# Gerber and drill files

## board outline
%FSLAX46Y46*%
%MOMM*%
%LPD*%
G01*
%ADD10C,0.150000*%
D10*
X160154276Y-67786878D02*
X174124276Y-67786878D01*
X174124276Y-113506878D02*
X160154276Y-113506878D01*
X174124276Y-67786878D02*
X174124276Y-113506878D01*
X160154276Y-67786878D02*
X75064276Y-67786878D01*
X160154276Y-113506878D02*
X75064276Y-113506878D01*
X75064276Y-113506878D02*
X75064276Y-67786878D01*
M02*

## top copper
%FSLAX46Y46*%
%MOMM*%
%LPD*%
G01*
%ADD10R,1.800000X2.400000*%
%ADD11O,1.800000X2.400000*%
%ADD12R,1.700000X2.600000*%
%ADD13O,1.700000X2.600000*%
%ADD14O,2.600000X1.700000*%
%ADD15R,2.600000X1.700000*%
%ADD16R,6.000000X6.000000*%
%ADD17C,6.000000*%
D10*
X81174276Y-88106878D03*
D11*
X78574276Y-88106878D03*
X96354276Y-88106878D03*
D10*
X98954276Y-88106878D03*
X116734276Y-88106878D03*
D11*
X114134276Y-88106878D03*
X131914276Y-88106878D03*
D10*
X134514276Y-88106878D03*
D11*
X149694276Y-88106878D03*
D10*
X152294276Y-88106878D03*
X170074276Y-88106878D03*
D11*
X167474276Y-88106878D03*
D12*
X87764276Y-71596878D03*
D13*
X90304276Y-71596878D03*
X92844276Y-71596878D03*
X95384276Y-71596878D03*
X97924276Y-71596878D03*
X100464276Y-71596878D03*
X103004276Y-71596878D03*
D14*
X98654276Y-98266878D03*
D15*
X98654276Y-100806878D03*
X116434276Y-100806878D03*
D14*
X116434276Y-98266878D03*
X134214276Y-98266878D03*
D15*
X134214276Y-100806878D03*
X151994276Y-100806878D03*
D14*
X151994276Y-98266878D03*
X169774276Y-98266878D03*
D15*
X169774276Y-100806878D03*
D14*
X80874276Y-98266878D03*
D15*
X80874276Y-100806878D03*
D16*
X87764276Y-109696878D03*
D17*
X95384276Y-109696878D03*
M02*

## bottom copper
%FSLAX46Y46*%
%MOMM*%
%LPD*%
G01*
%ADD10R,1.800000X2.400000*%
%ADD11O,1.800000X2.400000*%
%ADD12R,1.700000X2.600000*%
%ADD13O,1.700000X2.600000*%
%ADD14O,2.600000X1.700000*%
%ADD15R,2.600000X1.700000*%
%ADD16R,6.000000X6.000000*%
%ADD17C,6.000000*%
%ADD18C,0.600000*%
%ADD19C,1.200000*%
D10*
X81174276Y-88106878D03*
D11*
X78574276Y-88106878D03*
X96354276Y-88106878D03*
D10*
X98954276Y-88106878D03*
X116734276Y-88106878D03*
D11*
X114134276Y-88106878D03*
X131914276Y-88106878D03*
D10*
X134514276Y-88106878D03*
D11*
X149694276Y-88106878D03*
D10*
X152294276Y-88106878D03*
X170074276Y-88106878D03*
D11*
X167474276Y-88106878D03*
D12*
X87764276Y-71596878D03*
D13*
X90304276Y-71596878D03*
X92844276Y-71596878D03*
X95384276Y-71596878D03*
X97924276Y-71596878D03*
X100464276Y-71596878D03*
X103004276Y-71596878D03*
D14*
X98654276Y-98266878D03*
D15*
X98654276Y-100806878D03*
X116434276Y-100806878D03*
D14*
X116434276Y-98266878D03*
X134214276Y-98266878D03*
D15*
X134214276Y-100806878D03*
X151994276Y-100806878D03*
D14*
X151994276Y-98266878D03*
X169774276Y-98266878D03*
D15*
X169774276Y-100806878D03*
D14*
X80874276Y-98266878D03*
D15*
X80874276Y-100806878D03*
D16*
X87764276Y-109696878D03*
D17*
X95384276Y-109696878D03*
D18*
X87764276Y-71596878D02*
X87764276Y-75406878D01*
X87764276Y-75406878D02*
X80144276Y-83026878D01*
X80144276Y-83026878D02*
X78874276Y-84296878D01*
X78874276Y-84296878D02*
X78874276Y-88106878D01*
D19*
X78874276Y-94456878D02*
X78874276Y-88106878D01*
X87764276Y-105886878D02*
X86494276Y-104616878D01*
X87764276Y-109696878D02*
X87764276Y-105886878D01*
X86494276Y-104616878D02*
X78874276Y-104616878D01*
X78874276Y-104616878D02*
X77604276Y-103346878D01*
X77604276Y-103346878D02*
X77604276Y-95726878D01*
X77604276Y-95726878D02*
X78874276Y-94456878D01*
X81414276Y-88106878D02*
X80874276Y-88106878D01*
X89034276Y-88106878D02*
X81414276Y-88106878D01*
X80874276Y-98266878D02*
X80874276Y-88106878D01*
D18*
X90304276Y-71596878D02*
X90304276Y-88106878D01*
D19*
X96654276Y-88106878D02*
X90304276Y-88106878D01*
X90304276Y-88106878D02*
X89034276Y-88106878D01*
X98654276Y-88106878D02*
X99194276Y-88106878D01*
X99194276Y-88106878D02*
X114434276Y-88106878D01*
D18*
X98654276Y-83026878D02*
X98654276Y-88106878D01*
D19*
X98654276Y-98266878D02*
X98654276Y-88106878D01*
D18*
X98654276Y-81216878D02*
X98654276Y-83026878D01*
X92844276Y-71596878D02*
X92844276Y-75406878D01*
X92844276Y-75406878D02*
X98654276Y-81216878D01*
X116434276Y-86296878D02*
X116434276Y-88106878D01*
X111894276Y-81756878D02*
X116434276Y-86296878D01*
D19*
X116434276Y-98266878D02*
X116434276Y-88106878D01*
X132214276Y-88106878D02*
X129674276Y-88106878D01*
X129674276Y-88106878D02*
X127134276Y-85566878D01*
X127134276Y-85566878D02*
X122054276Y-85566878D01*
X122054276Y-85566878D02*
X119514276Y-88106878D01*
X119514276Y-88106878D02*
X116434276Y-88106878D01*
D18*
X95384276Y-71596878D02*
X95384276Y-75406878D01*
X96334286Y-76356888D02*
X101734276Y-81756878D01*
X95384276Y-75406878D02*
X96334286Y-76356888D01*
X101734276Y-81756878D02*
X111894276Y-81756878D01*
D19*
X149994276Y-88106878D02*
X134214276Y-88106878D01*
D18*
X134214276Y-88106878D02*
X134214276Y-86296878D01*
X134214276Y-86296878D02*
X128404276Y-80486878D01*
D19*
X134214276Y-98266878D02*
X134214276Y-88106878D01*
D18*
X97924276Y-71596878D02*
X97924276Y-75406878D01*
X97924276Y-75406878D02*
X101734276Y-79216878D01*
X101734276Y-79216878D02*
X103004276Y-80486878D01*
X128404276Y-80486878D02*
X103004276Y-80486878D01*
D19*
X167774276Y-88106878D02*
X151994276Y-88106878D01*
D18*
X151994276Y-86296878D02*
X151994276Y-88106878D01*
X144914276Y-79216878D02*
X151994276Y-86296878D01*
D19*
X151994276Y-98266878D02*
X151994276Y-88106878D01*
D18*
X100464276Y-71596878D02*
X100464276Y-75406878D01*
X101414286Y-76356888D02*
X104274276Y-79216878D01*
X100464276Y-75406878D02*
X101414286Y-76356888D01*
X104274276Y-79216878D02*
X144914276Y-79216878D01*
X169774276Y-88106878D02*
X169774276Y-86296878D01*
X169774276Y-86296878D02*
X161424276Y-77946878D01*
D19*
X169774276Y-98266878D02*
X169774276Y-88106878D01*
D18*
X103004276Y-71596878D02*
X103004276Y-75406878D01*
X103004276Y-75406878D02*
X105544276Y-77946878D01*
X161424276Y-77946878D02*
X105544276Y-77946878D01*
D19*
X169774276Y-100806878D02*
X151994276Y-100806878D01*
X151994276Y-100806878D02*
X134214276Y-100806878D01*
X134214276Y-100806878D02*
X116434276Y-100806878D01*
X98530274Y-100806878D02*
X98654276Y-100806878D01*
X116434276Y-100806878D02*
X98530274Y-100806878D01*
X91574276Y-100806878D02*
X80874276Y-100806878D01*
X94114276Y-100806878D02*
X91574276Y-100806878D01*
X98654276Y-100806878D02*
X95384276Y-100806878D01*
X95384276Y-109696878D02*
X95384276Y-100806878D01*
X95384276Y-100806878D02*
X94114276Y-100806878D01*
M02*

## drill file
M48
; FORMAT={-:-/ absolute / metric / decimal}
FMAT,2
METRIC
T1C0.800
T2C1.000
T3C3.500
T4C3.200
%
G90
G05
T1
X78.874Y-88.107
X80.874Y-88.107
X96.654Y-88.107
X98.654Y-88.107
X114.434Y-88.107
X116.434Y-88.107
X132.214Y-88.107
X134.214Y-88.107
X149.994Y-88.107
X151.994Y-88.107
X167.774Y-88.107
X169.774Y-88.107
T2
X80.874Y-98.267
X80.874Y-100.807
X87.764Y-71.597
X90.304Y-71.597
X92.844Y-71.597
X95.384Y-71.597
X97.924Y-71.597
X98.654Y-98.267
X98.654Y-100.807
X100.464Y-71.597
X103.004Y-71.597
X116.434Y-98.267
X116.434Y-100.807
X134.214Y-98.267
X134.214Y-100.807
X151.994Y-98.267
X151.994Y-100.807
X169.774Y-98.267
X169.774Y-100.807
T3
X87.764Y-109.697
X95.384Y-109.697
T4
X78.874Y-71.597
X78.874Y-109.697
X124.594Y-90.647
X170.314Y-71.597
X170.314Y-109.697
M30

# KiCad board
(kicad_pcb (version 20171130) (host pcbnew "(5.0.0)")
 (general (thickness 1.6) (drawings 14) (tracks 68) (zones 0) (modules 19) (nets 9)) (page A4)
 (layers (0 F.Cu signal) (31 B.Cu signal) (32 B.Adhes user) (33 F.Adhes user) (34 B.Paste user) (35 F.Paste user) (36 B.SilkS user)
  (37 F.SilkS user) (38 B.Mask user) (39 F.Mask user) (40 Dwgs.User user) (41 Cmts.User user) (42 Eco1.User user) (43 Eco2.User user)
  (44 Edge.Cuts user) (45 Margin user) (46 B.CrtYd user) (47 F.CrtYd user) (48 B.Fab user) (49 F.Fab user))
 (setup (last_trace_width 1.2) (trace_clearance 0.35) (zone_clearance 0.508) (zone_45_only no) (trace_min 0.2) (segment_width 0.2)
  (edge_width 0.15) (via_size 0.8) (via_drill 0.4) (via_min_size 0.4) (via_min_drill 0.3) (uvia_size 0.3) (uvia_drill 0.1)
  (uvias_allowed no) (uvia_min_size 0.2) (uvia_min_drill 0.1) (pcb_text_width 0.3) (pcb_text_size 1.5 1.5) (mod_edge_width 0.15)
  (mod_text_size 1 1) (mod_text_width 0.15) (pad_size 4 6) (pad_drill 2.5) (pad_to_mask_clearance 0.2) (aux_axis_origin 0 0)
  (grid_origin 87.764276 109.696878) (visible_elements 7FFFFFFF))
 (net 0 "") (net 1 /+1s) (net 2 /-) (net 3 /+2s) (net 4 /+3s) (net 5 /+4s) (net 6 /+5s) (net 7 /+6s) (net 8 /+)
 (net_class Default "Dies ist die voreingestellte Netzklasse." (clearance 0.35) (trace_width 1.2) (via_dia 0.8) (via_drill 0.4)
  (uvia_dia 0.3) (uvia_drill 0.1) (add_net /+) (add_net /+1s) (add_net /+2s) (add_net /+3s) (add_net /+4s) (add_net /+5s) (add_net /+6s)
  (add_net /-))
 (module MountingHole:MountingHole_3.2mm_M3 (layer F.Cu) (at 124.594276 90.646878 90)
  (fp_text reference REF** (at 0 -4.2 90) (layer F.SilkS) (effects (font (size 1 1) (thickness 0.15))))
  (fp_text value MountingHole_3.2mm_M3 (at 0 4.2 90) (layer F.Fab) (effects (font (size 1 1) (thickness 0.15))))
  (pad 1 np_thru_hole circle (at 0 0 90) (size 3.2 3.2) (drill 3.2) (layers *.Cu *.Mask)))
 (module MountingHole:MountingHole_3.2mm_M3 (layer F.Cu) (at 170.314276 109.696878 90)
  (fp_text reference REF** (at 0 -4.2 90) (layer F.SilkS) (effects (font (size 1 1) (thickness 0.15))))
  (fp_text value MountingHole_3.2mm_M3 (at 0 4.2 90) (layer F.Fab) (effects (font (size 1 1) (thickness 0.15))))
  (pad 1 np_thru_hole circle (at 0 0 90) (size 3.2 3.2) (drill 3.2) (layers *.Cu *.Mask)))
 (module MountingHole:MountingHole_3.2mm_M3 (layer F.Cu) (at 170.314276 71.596878 90)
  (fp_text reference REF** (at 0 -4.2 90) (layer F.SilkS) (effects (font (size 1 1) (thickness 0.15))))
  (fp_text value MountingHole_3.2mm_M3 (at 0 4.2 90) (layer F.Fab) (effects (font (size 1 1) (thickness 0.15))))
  (pad 1 np_thru_hole circle (at 0 0 90) (size 3.2 3.2) (drill 3.2) (layers *.Cu *.Mask)))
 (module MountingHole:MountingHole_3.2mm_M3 (layer F.Cu) (at 78.874276 109.696878 90)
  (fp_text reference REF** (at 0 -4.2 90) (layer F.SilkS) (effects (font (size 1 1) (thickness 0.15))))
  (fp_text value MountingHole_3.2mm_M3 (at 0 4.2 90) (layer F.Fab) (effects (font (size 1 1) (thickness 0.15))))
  (pad 1 np_thru_hole circle (at 0 0 90) (size 3.2 3.2) (drill 3.2) (layers *.Cu *.Mask)))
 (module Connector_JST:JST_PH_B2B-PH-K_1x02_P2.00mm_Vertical (layer F.Cu) (at 80.874276 88.106878 180)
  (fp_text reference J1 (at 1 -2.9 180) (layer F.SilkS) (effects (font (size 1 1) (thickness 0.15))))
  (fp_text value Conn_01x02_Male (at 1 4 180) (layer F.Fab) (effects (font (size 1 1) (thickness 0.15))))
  (pad 1 thru_hole rect (at 0 0 180) (size 1.8 2.4) (drill 0.8 (offset -0.3 0)) (layers *.Cu *.Mask) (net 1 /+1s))
  (pad 2 thru_hole oval (at 2 0 180) (size 1.8 2.4) (drill 0.8 (offset 0.3 0)) (layers *.Cu *.Mask) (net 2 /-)))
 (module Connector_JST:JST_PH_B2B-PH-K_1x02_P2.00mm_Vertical (layer F.Cu) (at 98.654276 88.106878 180)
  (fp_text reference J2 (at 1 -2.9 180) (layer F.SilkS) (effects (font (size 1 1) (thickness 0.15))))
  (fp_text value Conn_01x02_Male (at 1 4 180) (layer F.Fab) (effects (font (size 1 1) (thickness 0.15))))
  (pad 2 thru_hole oval (at 2 0 180) (size 1.8 2.4) (drill 0.8 (offset 0.3 0)) (layers *.Cu *.Mask) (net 1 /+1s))
  (pad 1 thru_hole rect (at 0 0 180) (size 1.8 2.4) (drill 0.8 (offset -0.3 0)) (layers *.Cu *.Mask) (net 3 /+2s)))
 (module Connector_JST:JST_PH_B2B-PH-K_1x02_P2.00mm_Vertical (layer F.Cu) (at 116.434276 88.106878 180)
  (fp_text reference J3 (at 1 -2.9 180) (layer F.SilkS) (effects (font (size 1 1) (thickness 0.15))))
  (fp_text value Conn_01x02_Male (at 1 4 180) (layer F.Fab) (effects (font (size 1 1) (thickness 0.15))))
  (pad 1 thru_hole rect (at 0 0 180) (size 1.8 2.4) (drill 0.8 (offset -0.3 0)) (layers *.Cu *.Mask) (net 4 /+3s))
  (pad 2 thru_hole oval (at 2 0 180) (size 1.8 2.4) (drill 0.8 (offset 0.3 0)) (layers *.Cu *.Mask) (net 3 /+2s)))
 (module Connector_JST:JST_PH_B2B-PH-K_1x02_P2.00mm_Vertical (layer F.Cu) (at 134.214276 88.106878 180)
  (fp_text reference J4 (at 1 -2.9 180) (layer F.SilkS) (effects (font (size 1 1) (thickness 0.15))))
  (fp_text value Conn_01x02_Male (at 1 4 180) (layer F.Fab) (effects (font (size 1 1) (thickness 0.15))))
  (pad 2 thru_hole oval (at 2 0 180) (size 1.8 2.4) (drill 0.8 (offset 0.3 0)) (layers *.Cu *.Mask) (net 4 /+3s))
  (pad 1 thru_hole rect (at 0 0 180) (size 1.8 2.4) (drill 0.8 (offset -0.3 0)) (layers *.Cu *.Mask) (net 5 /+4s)))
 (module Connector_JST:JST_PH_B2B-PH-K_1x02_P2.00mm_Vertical (layer F.Cu) (at 151.994276 88.106878 180)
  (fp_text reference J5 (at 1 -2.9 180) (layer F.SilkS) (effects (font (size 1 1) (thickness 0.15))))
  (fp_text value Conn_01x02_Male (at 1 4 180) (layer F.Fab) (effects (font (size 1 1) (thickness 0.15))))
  (pad 2 thru_hole oval (at 2 0 180) (size 1.8 2.4) (drill 0.8 (offset 0.3 0)) (layers *.Cu *.Mask) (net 5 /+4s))
  (pad 1 thru_hole rect (at 0 0 180) (size 1.8 2.4) (drill 0.8 (offset -0.3 0)) (layers *.Cu *.Mask) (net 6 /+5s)))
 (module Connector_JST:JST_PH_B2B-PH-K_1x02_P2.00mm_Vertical (layer F.Cu) (at 169.774276 88.106878 180)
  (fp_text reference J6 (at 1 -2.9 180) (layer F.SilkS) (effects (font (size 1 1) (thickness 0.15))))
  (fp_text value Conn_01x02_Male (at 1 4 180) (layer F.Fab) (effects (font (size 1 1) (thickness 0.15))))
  (pad 1 thru_hole rect (at 0 0 180) (size 1.8 2.4) (drill 0.8 (offset -0.3 0)) (layers *.Cu *.Mask) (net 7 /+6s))
  (pad 2 thru_hole oval (at 2 0 180) (size 1.8 2.4) (drill 0.8 (offset 0.3 0)) (layers *.Cu *.Mask) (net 6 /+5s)))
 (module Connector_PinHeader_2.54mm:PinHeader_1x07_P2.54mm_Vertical (layer F.Cu) (at 87.764276 71.596878 90)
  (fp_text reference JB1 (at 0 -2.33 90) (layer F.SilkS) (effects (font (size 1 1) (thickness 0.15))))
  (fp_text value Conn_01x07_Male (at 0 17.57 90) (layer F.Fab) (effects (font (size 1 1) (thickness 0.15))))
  (pad 1 thru_hole rect (at 0 0 90) (size 2.6 1.7) (drill 1) (layers *.Cu *.Mask) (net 2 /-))
  (pad 2 thru_hole oval (at 0 2.54 90) (size 2.6 1.7) (drill 1) (layers *.Cu *.Mask) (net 1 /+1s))
  (pad 3 thru_hole oval (at 0 5.08 90) (size 2.6 1.7) (drill 1) (layers *.Cu *.Mask) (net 3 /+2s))
  (pad 4 thru_hole oval (at 0 7.62 90) (size 2.6 1.7) (drill 1) (layers *.Cu *.Mask) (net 4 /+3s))
  (pad 5 thru_hole oval (at 0 10.16 90) (size 2.6 1.7) (drill 1) (layers *.Cu *.Mask) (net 5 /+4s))
  (pad 6 thru_hole oval (at 0 12.7 90) (size 2.6 1.7) (drill 1) (layers *.Cu *.Mask) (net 6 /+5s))
  (pad 7 thru_hole oval (at 0 15.24 90) (size 2.6 1.7) (drill 1) (layers *.Cu *.Mask) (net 7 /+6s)))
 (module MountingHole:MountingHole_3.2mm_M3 (layer F.Cu) (at 78.874276 71.596878 90)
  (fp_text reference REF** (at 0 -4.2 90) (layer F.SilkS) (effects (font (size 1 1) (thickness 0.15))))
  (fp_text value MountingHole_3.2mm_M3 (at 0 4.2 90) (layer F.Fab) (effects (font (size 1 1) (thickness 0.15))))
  (pad 1 np_thru_hole circle (at 0 0 90) (size 3.2 3.2) (drill 3.2) (layers *.Cu *.Mask)))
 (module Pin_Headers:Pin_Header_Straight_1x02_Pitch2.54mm (layer F.Cu) (at 98.654276 100.806878 180)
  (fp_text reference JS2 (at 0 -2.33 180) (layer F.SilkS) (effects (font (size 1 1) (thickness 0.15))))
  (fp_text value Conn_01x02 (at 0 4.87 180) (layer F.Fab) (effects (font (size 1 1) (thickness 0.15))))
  (pad 2 thru_hole oval (at 0 2.54 180) (size 2.6 1.7) (drill 1) (layers *.Cu *.Mask) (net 3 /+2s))
  (pad 1 thru_hole rect (at 0 0 180) (size 2.6 1.7) (drill 1) (layers *.Cu *.Mask) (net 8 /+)))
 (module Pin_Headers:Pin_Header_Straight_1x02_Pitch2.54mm (layer F.Cu) (at 116.434276 100.806878 180)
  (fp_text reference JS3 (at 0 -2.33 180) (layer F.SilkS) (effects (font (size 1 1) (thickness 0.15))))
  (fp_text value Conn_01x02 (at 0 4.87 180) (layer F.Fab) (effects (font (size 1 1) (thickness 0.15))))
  (pad 1 thru_hole rect (at 0 0 180) (size 2.6 1.7) (drill 1) (layers *.Cu *.Mask) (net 8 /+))
  (pad 2 thru_hole oval (at 0 2.54 180) (size 2.6 1.7) (drill 1) (layers *.Cu *.Mask) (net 4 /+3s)))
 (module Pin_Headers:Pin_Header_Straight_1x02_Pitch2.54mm (layer F.Cu) (at 134.214276 100.806878 180)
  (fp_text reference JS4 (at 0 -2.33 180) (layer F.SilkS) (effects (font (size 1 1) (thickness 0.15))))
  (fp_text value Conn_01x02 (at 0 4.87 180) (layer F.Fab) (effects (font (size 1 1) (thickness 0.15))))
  (pad 2 thru_hole oval (at 0 2.54 180) (size 2.6 1.7) (drill 1) (layers *.Cu *.Mask) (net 5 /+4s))
  (pad 1 thru_hole rect (at 0 0 180) (size 2.6 1.7) (drill 1) (layers *.Cu *.Mask) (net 8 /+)))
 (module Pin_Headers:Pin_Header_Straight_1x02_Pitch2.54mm (layer F.Cu) (at 151.994276 100.806878 180)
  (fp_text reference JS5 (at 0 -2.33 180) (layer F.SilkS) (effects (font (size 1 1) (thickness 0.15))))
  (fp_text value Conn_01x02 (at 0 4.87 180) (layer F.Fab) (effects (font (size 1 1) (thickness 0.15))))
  (pad 1 thru_hole rect (at 0 0 180) (size 2.6 1.7) (drill 1) (layers *.Cu *.Mask) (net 8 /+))
  (pad 2 thru_hole oval (at 0 2.54 180) (size 2.6 1.7) (drill 1) (layers *.Cu *.Mask) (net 6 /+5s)))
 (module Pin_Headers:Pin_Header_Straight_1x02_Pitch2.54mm (layer F.Cu) (at 169.774276 100.806878 180)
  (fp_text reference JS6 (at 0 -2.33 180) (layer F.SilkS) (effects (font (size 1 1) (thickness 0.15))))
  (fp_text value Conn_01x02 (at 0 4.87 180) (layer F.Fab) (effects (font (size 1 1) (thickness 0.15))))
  (pad 2 thru_hole oval (at 0 2.54 180) (size 2.6 1.7) (drill 1) (layers *.Cu *.Mask) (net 7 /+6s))
  (pad 1 thru_hole rect (at 0 0 180) (size 2.6 1.7) (drill 1) (layers *.Cu *.Mask) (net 8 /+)))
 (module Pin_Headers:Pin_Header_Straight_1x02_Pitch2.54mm (layer F.Cu) (at 80.874276 100.806878 180)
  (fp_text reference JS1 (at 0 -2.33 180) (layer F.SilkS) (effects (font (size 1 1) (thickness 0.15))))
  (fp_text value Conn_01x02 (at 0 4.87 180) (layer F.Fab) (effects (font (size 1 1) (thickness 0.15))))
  (pad 2 thru_hole oval (at 0 2.54 180) (size 2.6 1.7) (drill 1) (layers *.Cu *.Mask) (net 1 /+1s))
  (pad 1 thru_hole rect (at 0 0 180) (size 2.6 1.7) (drill 1) (layers *.Cu *.Mask) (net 8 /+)))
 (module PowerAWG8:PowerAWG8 (layer F.Cu) (at 87.764276 109.696878)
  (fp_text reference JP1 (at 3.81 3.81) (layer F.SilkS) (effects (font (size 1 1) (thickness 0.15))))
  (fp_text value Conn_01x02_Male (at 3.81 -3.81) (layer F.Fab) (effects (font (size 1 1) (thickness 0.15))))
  (pad 1 thru_hole rect (at 0 0) (size 6 6) (drill 3.5) (layers *.Cu *.Mask) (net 2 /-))
  (pad 2 thru_hole circle (at 7.62 0) (size 6 6) (drill 3.5) (layers *.Cu *.Mask) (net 8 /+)))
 (gr_line (start 160.154276 67.786878) (end 174.124276 67.786878) (layer Edge.Cuts) (width 0.15))
 (gr_line (start 174.124276 113.506878) (end 160.154276 113.506878) (layer Edge.Cuts) (width 0.15))
 (gr_line (start 174.124276 67.786878) (end 174.124276 113.506878) (layer Edge.Cuts) (width 0.15))
 (gr_line (start 160.154276 67.786878) (end 75.064276 67.786878) (layer Edge.Cuts) (width 0.15))
 (gr_line (start 160.154276 113.506878) (end 75.064276 113.506878) (layer Edge.Cuts) (width 0.15))
 (gr_line (start 75.064276 113.506878) (end 75.064276 67.786878) (layer Edge.Cuts) (width 0.15))
 (segment (start 87.764276 71.596878) (end 87.764276 75.406878) (width 0.6) (layer B.Cu) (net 2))
 (segment (start 87.764276 75.406878) (end 80.144276 83.026878) (width 0.6) (layer B.Cu) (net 2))
 (segment (start 80.144276 83.026878) (end 78.874276 84.296878) (width 0.6) (layer B.Cu) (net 2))
 (segment (start 78.874276 84.296878) (end 78.874276 88.106878) (width 0.6) (layer B.Cu) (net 2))
 (segment (start 78.874276 94.456878) (end 78.874276 88.106878) (width 1.2) (layer B.Cu) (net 2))
 (segment (start 87.764276 105.886878) (end 86.494276 104.616878) (width 1.2) (layer B.Cu) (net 2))
 (segment (start 87.764276 109.696878) (end 87.764276 105.886878) (width 1.2) (layer B.Cu) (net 2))
 (segment (start 86.494276 104.616878) (end 78.874276 104.616878) (width 1.2) (layer B.Cu) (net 2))
 (segment (start 78.874276 104.616878) (end 77.604276 103.346878) (width 1.2) (layer B.Cu) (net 2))
 (segment (start 77.604276 103.346878) (end 77.604276 95.726878) (width 1.2) (layer B.Cu) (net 2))
 (segment (start 77.604276 95.726878) (end 78.874276 94.456878) (width 1.2) (layer B.Cu) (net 2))
 (segment (start 81.414276 88.106878) (end 80.874276 88.106878) (width 1.2) (layer B.Cu) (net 1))
 (segment (start 89.034276 88.106878) (end 81.414276 88.106878) (width 1.2) (layer B.Cu) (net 1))
 (segment (start 80.874276 98.266878) (end 80.874276 88.106878) (width 1.2) (layer B.Cu) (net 1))
 (segment (start 90.304276 71.596878) (end 90.304276 88.106878) (width 0.6) (layer B.Cu) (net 1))
 (segment (start 96.654276 88.106878) (end 90.304276 88.106878) (width 1.2) (layer B.Cu) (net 1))
 (segment (start 90.304276 88.106878) (end 89.034276 88.106878) (width 1.2) (layer B.Cu) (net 1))
 (segment (start 98.654276 88.106878) (end 99.194276 88.106878) (width 1.2) (layer B.Cu) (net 3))
 (segment (start 99.194276 88.106878) (end 114.434276 88.106878) (width 1.2) (layer B.Cu) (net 3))
 (segment (start 98.654276 83.026878) (end 98.654276 88.106878) (width 0.6) (layer B.Cu) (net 3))
 (segment (start 98.654276 98.266878) (end 98.654276 88.106878) (width 1.2) (layer B.Cu) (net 3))
 (segment (start 98.654276 81.216878) (end 98.654276 83.026878) (width 0.6) (layer B.Cu) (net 3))
 (segment (start 92.844276 71.596878) (end 92.844276 75.406878) (width 0.6) (layer B.Cu) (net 3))
 (segment (start 92.844276 75.406878) (end 98.654276 81.216878) (width 0.6) (layer B.Cu) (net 3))
 (segment (start 116.434276 86.296878) (end 116.434276 88.106878) (width 0.6) (layer B.Cu) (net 4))
 (segment (start 111.894276 81.756878) (end 116.434276 86.296878) (width 0.6) (layer B.Cu) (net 4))
 (segment (start 116.434276 98.266878) (end 116.434276 88.106878) (width 1.2) (layer B.Cu) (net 4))
 (segment (start 132.214276 88.106878) (end 129.674276 88.106878) (width 1.2) (layer B.Cu) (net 4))
 (segment (start 129.674276 88.106878) (end 127.134276 85.566878) (width 1.2) (layer B.Cu) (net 4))
 (segment (start 127.134276 85.566878) (end 122.054276 85.566878) (width 1.2) (layer B.Cu) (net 4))
 (segment (start 122.054276 85.566878) (end 119.514276 88.106878) (width 1.2) (layer B.Cu) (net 4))
 (segment (start 119.514276 88.106878) (end 116.434276 88.106878) (width 1.2) (layer B.Cu) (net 4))
 (segment (start 95.384276 71.596878) (end 95.384276 75.406878) (width 0.6) (layer B.Cu) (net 4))
 (segment (start 96.334286 76.356888) (end 101.734276 81.756878) (width 0.6) (layer B.Cu) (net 4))
 (segment (start 95.384276 75.406878) (end 96.334286 76.356888) (width 0.6) (layer B.Cu) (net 4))
 (segment (start 101.734276 81.756878) (end 111.894276 81.756878) (width 0.6) (layer B.Cu) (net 4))
 (segment (start 149.994276 88.106878) (end 134.214276 88.106878) (width 1.2) (layer B.Cu) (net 5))
 (segment (start 134.214276 88.106878) (end 134.214276 86.296878) (width 0.6) (layer B.Cu) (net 5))
 (segment (start 134.214276 86.296878) (end 128.404276 80.486878) (width 0.6) (layer B.Cu) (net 5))
 (segment (start 134.214276 98.266878) (end 134.214276 88.106878) (width 1.2) (layer B.Cu) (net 5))
 (segment (start 97.924276 71.596878) (end 97.924276 75.406878) (width 0.6) (layer B.Cu) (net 5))
 (segment (start 97.924276 75.406878) (end 101.734276 79.216878) (width 0.6) (layer B.Cu) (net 5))
 (segment (start 101.734276 79.216878) (end 103.004276 80.486878) (width 0.6) (layer B.Cu) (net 5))
 (segment (start 128.404276 80.486878) (end 103.004276 80.486878) (width 0.6) (layer B.Cu) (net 5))
 (segment (start 167.774276 88.106878) (end 151.994276 88.106878) (width 1.2) (layer B.Cu) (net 6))
 (segment (start 151.994276 86.296878) (end 151.994276 88.106878) (width 0.6) (layer B.Cu) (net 6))
 (segment (start 144.914276 79.216878) (end 151.994276 86.296878) (width 0.6) (layer B.Cu) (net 6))
 (segment (start 151.994276 98.266878) (end 151.994276 88.106878) (width 1.2) (layer B.Cu) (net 6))
 (segment (start 100.464276 71.596878) (end 100.464276 75.406878) (width 0.6) (layer B.Cu) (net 6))
 (segment (start 101.414286 76.356888) (end 104.274276 79.216878) (width 0.6) (layer B.Cu) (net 6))
 (segment (start 100.464276 75.406878) (end 101.414286 76.356888) (width 0.6) (layer B.Cu) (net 6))
 (segment (start 104.274276 79.216878) (end 144.914276 79.216878) (width 0.6) (layer B.Cu) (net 6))
 (segment (start 169.774276 88.106878) (end 169.774276 86.296878) (width 0.6) (layer B.Cu) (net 7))
 (segment (start 169.774276 86.296878) (end 161.424276 77.946878) (width 0.6) (layer B.Cu) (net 7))
 (segment (start 169.774276 98.266878) (end 169.774276 88.106878) (width 1.2) (layer B.Cu) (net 7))
 (segment (start 103.004276 71.596878) (end 103.004276 75.406878) (width 0.6) (layer B.Cu) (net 7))
 (segment (start 103.004276 75.406878) (end 105.544276 77.946878) (width 0.6) (layer B.Cu) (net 7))
 (segment (start 161.424276 77.946878) (end 105.544276 77.946878) (width 0.6) (layer B.Cu) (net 7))
 (segment (start 169.774276 100.806878) (end 151.994276 100.806878) (width 1.2) (layer B.Cu) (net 8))
 (segment (start 151.994276 100.806878) (end 134.214276 100.806878) (width 1.2) (layer B.Cu) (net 8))
 (segment (start 134.214276 100.806878) (end 116.434276 100.806878) (width 1.2) (layer B.Cu) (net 8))
 (segment (start 98.530274 100.806878) (end 98.654276 100.806878) (width 1.2) (layer B.Cu) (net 8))
 (segment (start 116.434276 100.806878) (end 98.530274 100.806878) (width 1.2) (layer B.Cu) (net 8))
 (segment (start 91.574276 100.806878) (end 80.874276 100.806878) (width 1.2) (layer B.Cu) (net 8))
 (segment (start 94.114276 100.806878) (end 91.574276 100.806878) (width 1.2) (layer B.Cu) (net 8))
 (segment (start 98.654276 100.806878) (end 95.384276 100.806878) (width 1.2) (layer B.Cu) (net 8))
 (segment (start 95.384276 109.696878) (end 95.384276 100.806878) (width 1.2) (layer B.Cu) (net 8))
 (segment (start 95.384276 100.806878) (end 94.114276 100.806878) (width 1.2) (layer B.Cu) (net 8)))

